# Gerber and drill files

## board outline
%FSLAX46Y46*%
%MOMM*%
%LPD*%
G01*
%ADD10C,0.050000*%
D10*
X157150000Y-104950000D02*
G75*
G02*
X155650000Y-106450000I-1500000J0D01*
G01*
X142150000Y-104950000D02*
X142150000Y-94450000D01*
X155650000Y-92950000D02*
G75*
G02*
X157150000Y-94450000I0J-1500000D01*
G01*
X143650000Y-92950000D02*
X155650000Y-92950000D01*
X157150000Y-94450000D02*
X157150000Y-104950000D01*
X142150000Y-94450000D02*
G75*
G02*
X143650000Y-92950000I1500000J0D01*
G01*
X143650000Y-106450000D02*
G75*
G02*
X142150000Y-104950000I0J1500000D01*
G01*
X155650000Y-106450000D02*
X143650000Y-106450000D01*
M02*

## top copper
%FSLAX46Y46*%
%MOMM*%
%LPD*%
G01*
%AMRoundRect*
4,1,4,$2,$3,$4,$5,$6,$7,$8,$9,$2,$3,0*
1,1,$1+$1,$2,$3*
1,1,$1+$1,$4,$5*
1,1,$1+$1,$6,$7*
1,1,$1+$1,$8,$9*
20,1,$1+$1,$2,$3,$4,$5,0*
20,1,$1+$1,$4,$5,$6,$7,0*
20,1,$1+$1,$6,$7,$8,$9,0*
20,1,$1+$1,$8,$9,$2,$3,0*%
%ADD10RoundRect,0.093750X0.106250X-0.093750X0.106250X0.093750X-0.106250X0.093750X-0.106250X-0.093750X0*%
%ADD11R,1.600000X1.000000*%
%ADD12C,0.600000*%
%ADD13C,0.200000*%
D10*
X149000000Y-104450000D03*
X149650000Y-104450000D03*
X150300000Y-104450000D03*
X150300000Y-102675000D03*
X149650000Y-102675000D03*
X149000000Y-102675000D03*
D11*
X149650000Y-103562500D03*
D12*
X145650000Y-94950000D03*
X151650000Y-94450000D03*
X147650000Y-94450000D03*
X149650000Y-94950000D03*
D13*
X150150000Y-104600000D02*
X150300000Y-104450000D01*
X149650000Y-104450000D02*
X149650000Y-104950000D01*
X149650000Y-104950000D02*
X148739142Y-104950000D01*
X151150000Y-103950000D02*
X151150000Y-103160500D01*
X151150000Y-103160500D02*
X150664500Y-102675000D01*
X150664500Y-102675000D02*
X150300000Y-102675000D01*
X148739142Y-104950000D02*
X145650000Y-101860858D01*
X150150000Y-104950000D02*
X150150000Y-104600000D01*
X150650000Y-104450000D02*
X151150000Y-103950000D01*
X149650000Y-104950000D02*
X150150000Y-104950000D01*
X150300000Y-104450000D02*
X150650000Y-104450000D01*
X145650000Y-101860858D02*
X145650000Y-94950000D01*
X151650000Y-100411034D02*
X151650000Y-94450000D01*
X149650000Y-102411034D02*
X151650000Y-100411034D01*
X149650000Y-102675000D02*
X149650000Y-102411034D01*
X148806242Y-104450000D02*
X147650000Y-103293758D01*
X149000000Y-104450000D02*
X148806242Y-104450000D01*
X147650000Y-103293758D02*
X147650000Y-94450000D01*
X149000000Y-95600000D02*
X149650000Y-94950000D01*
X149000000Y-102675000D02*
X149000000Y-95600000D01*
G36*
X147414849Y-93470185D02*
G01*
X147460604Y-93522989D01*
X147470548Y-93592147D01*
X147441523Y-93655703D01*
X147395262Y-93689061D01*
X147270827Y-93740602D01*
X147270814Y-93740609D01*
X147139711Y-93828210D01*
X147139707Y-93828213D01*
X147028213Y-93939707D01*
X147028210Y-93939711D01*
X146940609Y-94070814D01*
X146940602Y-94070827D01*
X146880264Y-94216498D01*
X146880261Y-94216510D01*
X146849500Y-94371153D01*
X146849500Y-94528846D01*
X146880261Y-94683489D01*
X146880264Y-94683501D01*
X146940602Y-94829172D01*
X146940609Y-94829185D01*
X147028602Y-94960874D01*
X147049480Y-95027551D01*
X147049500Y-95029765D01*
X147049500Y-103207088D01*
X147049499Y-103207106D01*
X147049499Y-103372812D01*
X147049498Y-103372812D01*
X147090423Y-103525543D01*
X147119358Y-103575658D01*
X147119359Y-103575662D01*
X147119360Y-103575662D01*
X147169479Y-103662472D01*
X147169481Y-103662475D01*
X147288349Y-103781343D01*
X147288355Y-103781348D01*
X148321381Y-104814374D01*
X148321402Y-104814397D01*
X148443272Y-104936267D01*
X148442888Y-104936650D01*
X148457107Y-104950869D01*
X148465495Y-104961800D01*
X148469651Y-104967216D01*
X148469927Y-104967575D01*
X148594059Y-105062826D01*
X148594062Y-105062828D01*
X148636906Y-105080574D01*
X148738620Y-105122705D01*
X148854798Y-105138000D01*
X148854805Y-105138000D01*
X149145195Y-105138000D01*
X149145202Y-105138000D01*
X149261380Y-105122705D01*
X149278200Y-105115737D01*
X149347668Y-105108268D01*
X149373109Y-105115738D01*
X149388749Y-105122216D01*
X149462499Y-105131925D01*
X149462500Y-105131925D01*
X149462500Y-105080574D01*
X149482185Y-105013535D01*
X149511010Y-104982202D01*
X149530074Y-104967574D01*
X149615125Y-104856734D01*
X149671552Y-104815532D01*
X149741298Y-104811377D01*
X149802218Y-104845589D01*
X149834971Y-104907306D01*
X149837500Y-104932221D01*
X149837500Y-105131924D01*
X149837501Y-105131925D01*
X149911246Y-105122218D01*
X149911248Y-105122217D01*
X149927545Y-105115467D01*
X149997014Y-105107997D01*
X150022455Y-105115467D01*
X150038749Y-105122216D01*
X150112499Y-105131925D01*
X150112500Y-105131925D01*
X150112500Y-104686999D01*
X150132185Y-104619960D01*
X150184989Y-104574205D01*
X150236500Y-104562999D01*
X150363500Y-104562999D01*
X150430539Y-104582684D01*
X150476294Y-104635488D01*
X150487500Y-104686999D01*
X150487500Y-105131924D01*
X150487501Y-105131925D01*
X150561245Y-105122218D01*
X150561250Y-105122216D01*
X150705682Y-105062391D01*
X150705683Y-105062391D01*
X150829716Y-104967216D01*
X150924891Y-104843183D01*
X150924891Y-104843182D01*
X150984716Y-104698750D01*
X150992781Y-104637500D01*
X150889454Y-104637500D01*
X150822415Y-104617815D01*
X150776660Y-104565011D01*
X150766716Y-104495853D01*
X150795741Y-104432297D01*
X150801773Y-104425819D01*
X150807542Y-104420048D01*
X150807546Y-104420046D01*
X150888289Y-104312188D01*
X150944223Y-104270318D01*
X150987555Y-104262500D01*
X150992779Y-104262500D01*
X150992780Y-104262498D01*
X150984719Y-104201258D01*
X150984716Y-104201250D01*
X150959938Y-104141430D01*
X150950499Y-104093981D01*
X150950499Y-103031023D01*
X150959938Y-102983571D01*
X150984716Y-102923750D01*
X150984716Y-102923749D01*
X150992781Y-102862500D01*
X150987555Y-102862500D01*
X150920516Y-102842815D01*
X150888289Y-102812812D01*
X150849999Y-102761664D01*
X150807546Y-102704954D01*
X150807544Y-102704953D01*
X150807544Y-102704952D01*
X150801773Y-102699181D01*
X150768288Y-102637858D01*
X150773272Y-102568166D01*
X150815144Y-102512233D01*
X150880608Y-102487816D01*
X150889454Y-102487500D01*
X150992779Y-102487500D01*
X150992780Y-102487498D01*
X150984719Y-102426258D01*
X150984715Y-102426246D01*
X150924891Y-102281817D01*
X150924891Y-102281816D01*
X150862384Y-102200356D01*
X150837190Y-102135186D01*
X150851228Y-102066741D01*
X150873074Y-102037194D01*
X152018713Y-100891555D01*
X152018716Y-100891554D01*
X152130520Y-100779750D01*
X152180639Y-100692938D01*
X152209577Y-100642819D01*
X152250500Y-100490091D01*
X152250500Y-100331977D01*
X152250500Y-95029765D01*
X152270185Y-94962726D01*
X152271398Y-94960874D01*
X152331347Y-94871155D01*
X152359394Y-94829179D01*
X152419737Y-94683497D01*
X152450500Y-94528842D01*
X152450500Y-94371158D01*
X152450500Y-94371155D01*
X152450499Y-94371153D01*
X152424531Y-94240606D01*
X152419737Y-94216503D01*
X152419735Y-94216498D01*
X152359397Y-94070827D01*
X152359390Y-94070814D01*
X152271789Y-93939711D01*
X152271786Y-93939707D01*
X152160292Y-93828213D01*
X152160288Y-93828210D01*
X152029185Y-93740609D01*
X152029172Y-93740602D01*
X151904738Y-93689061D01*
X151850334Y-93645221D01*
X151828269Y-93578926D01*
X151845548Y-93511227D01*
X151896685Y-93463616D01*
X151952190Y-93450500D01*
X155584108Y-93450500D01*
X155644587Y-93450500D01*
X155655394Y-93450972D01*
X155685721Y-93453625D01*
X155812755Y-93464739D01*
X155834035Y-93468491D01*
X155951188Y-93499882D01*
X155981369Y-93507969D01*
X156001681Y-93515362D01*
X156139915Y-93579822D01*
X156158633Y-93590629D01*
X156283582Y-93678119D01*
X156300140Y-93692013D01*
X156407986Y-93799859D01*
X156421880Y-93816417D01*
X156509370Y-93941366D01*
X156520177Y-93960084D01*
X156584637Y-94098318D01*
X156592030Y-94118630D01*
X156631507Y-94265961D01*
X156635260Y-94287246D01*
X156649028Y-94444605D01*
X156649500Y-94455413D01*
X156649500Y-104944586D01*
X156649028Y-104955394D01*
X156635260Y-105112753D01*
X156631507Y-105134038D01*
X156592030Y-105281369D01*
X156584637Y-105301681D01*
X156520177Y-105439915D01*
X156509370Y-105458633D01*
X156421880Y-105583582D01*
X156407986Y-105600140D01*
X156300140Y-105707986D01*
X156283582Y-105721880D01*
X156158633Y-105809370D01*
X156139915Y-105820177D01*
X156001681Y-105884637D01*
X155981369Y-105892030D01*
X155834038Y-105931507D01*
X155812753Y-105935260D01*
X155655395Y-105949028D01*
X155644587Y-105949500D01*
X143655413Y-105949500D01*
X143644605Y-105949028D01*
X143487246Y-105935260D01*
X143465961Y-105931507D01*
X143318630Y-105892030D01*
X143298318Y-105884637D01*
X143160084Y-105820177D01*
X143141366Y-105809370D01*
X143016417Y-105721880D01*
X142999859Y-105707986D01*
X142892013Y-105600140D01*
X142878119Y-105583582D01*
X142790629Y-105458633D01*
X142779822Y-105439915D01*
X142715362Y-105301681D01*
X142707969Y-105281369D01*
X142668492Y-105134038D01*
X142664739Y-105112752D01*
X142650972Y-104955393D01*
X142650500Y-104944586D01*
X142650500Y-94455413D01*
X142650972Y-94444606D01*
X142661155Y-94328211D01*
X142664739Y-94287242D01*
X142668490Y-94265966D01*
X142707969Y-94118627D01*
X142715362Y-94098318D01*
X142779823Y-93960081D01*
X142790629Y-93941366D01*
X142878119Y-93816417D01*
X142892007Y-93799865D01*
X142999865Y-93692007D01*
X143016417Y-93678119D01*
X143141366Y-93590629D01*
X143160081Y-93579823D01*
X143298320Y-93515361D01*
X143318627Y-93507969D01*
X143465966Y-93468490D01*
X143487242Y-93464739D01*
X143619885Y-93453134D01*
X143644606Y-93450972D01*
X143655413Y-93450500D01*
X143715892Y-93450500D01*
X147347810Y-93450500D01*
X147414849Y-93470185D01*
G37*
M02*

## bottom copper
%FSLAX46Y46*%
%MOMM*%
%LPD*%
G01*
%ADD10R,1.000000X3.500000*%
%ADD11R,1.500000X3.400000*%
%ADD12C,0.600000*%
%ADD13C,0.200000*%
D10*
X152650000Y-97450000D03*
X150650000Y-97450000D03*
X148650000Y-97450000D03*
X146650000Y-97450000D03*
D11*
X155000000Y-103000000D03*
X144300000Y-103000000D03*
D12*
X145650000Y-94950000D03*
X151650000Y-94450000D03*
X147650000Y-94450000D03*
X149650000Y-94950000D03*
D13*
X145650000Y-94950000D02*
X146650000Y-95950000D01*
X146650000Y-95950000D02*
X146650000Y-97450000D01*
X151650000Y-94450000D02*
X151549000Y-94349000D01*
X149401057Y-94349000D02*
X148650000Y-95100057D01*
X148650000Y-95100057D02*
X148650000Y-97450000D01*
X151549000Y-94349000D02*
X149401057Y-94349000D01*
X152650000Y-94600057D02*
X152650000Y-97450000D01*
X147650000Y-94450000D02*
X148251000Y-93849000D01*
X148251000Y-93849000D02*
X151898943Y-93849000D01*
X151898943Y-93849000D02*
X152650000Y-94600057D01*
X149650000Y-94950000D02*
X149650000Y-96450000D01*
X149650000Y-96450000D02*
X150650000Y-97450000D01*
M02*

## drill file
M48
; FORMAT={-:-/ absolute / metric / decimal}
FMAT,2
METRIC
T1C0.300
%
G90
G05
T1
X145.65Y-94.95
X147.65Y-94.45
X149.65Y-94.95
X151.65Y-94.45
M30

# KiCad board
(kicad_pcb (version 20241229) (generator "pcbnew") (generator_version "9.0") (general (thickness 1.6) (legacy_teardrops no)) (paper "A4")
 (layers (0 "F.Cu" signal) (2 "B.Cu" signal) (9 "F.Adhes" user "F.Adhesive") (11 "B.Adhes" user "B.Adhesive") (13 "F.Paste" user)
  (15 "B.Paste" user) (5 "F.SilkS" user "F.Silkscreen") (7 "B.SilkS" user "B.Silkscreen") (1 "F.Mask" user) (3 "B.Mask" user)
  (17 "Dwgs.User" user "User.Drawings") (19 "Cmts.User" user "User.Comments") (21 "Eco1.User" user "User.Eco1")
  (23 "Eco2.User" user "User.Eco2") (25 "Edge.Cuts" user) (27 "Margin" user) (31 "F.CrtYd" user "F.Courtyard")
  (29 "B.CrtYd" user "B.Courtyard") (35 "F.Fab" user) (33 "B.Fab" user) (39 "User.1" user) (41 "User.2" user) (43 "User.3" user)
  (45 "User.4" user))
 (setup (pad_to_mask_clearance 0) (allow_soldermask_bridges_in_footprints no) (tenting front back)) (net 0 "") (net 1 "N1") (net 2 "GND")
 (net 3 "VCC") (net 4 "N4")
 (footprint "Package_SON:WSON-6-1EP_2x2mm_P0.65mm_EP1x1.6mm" (layer "F.Cu") (at 149.65 103.5625 90)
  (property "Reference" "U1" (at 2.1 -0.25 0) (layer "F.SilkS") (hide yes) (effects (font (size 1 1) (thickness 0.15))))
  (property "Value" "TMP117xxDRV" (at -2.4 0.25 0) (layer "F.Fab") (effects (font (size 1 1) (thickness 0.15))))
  (pad "" smd roundrect (at 0 -0.4 90) (size 0.81 0.64) (layers "F.Paste") (roundrect_rratio 0.25))
  (pad "" smd roundrect (at 0 0.4 90) (size 0.81 0.64) (layers "F.Paste") (roundrect_rratio 0.25))
  (pad "1" smd roundrect (at -0.8875 -0.65 90) (size 0.375 0.4) (layers "F.Cu" "F.Mask" "F.Paste") (roundrect_rratio 0.25) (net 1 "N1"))
  (pad "2" smd roundrect (at -0.8875 0 90) (size 0.375 0.4) (layers "F.Cu" "F.Mask" "F.Paste") (roundrect_rratio 0.25) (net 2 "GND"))
  (pad "3" smd roundrect (at -0.8875 0.65 90) (size 0.375 0.4) (layers "F.Cu" "F.Mask" "F.Paste") (roundrect_rratio 0.25) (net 2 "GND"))
  (pad "4" smd roundrect (at 0.8875 0.65 90) (size 0.375 0.4) (layers "F.Cu" "F.Mask" "F.Paste") (roundrect_rratio 0.25) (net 2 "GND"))
  (pad "5" smd roundrect (at 0.8875 0 90) (size 0.375 0.4) (layers "F.Cu" "F.Mask" "F.Paste") (roundrect_rratio 0.25) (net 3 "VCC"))
  (pad "6" smd roundrect (at 0.8875 -0.65 90) (size 0.375 0.4) (layers "F.Cu" "F.Mask" "F.Paste") (roundrect_rratio 0.25) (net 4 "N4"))
  (pad "7" smd rect (at 0 0 90) (size 1 1.6) (layers "F.Cu" "F.Mask") (zone_connect 2)))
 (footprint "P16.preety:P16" (layer "F.Cu") (at 154.15 102.95)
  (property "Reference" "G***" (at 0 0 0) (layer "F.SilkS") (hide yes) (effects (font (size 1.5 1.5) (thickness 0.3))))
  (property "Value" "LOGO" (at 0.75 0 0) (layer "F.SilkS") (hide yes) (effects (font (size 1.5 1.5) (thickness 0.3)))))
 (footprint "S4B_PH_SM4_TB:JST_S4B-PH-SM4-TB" (layer "B.Cu") (at 149.65 100.2 180)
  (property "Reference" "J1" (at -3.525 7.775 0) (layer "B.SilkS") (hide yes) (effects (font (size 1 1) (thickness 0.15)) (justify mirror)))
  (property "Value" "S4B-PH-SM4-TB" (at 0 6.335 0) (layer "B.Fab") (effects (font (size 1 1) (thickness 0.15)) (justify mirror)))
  (pad "1" smd rect (at -3 2.75 180) (size 1 3.5) (layers "B.Cu" "B.Mask" "B.Paste") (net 1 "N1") (solder_mask_margin 0.102))
  (pad "2" smd rect (at -1 2.75 180) (size 1 3.5) (layers "B.Cu" "B.Mask" "B.Paste") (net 4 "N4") (solder_mask_margin 0.102))
  (pad "3" smd rect (at 1 2.75 180) (size 1 3.5) (layers "B.Cu" "B.Mask" "B.Paste") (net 3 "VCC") (solder_mask_margin 0.102))
  (pad "4" smd rect (at 3 2.75 180) (size 1 3.5) (layers "B.Cu" "B.Mask" "B.Paste") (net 2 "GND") (solder_mask_margin 0.102))
  (pad "SH1" smd rect (at -5.35 -2.8 180) (size 1.5 3.4) (layers "B.Cu" "B.Mask" "B.Paste") (solder_mask_margin 0.102))
  (pad "SH2" smd rect (at 5.35 -2.8 180) (size 1.5 3.4) (layers "B.Cu" "B.Mask" "B.Paste") (solder_mask_margin 0.102)))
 (gr_arc (start 157.15 104.95) (mid 156.71066 106.01066) (end 155.65 106.45) (stroke (width 0.05) (type default)) (layer "Edge.Cuts"))
 (gr_line (start 142.15 104.95) (end 142.15 94.45) (stroke (width 0.05) (type default)) (layer "Edge.Cuts"))
 (gr_arc (start 155.65 92.95) (mid 156.71066 93.38934) (end 157.15 94.45) (stroke (width 0.05) (type default)) (layer "Edge.Cuts"))
 (gr_line (start 143.65 92.95) (end 155.65 92.95) (stroke (width 0.05) (type default)) (layer "Edge.Cuts"))
 (gr_line (start 157.15 94.45) (end 157.15 104.95) (stroke (width 0.05) (type default)) (layer "Edge.Cuts"))
 (gr_arc (start 142.15 94.45) (mid 142.58934 93.38934) (end 143.65 92.95) (stroke (width 0.05) (type default)) (layer "Edge.Cuts"))
 (gr_arc (start 143.65 106.45) (mid 142.58934 106.01066) (end 142.15 104.95) (stroke (width 0.05) (type default)) (layer "Edge.Cuts"))
 (gr_line (start 155.65 106.45) (end 143.65 106.45) (stroke (width 0.05) (type default)) (layer "Edge.Cuts"))
 (segment (start 150.15 104.6) (end 150.3 104.45) (width 0.2) (layer "F.Cu") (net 2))
 (segment (start 149.65 104.45) (end 149.65 104.95) (width 0.2) (layer "F.Cu") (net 2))
 (segment (start 149.65 104.95) (end 148.739142 104.95) (width 0.2) (layer "F.Cu") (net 2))
 (segment (start 151.15 103.95) (end 151.15 103.1605) (width 0.2) (layer "F.Cu") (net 2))
 (segment (start 151.15 103.1605) (end 150.6645 102.675) (width 0.2) (layer "F.Cu") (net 2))
 (segment (start 150.6645 102.675) (end 150.3 102.675) (width 0.2) (layer "F.Cu") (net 2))
 (segment (start 148.739142 104.95) (end 145.65 101.860858) (width 0.2) (layer "F.Cu") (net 2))
 (segment (start 150.15 104.95) (end 150.15 104.6) (width 0.2) (layer "F.Cu") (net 2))
 (segment (start 150.65 104.45) (end 151.15 103.95) (width 0.2) (layer "F.Cu") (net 2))
 (segment (start 149.65 104.95) (end 150.15 104.95) (width 0.2) (layer "F.Cu") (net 2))
 (segment (start 150.3 104.45) (end 150.65 104.45) (width 0.2) (layer "F.Cu") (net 2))
 (segment (start 145.65 101.860858) (end 145.65 94.95) (width 0.2) (layer "F.Cu") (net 2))
 (via (at 145.65 94.95) (size 0.6) (drill 0.3) (layers "F.Cu" "B.Cu") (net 2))
 (segment (start 145.65 94.95) (end 146.65 95.95) (width 0.2) (layer "B.Cu") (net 2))
 (segment (start 146.65 95.95) (end 146.65 97.45) (width 0.2) (layer "B.Cu") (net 2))
 (segment (start 151.65 100.411034) (end 151.65 94.45) (width 0.2) (layer "F.Cu") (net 3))
 (segment (start 149.65 102.411034) (end 151.65 100.411034) (width 0.2) (layer "F.Cu") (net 3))
 (segment (start 149.65 102.675) (end 149.65 102.411034) (width 0.2) (layer "F.Cu") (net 3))
 (via (at 151.65 94.45) (size 0.6) (drill 0.3) (layers "F.Cu" "B.Cu") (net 3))
 (segment (start 151.65 94.45) (end 151.549 94.349) (width 0.2) (layer "B.Cu") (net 3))
 (segment (start 149.401057 94.349) (end 148.65 95.100057) (width 0.2) (layer "B.Cu") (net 3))
 (segment (start 148.65 95.100057) (end 148.65 97.45) (width 0.2) (layer "B.Cu") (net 3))
 (segment (start 151.549 94.349) (end 149.401057 94.349) (width 0.2) (layer "B.Cu") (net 3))
 (segment (start 148.806242 104.45) (end 147.65 103.293758) (width 0.2) (layer "F.Cu") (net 1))
 (segment (start 149 104.45) (end 148.806242 104.45) (width 0.2) (layer "F.Cu") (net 1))
 (segment (start 147.65 103.293758) (end 147.65 94.45) (width 0.2) (layer "F.Cu") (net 1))
 (via (at 147.65 94.45) (size 0.6) (drill 0.3) (layers "F.Cu" "B.Cu") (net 1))
 (segment (start 152.65 94.600057) (end 152.65 97.45) (width 0.2) (layer "B.Cu") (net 1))
 (segment (start 147.65 94.45) (end 148.251 93.849) (width 0.2) (layer "B.Cu") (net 1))
 (segment (start 148.251 93.849) (end 151.898943 93.849) (width 0.2) (layer "B.Cu") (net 1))
 (segment (start 151.898943 93.849) (end 152.65 94.600057) (width 0.2) (layer "B.Cu") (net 1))
 (segment (start 149 95.6) (end 149.65 94.95) (width 0.2) (layer "F.Cu") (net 4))
 (segment (start 149 102.675) (end 149 95.6) (width 0.2) (layer "F.Cu") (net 4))
 (via (at 149.65 94.95) (size 0.6) (drill 0.3) (layers "F.Cu" "B.Cu") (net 4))
 (segment (start 149.65 94.95) (end 149.65 96.45) (width 0.2) (layer "B.Cu") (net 4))
 (segment (start 149.65 96.45) (end 150.65 97.45) (width 0.2) (layer "B.Cu") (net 4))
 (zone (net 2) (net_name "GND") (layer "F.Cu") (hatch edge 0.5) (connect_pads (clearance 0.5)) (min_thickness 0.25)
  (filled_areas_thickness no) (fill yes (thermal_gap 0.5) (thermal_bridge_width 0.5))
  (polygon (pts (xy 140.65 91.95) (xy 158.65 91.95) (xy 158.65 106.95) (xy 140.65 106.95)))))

